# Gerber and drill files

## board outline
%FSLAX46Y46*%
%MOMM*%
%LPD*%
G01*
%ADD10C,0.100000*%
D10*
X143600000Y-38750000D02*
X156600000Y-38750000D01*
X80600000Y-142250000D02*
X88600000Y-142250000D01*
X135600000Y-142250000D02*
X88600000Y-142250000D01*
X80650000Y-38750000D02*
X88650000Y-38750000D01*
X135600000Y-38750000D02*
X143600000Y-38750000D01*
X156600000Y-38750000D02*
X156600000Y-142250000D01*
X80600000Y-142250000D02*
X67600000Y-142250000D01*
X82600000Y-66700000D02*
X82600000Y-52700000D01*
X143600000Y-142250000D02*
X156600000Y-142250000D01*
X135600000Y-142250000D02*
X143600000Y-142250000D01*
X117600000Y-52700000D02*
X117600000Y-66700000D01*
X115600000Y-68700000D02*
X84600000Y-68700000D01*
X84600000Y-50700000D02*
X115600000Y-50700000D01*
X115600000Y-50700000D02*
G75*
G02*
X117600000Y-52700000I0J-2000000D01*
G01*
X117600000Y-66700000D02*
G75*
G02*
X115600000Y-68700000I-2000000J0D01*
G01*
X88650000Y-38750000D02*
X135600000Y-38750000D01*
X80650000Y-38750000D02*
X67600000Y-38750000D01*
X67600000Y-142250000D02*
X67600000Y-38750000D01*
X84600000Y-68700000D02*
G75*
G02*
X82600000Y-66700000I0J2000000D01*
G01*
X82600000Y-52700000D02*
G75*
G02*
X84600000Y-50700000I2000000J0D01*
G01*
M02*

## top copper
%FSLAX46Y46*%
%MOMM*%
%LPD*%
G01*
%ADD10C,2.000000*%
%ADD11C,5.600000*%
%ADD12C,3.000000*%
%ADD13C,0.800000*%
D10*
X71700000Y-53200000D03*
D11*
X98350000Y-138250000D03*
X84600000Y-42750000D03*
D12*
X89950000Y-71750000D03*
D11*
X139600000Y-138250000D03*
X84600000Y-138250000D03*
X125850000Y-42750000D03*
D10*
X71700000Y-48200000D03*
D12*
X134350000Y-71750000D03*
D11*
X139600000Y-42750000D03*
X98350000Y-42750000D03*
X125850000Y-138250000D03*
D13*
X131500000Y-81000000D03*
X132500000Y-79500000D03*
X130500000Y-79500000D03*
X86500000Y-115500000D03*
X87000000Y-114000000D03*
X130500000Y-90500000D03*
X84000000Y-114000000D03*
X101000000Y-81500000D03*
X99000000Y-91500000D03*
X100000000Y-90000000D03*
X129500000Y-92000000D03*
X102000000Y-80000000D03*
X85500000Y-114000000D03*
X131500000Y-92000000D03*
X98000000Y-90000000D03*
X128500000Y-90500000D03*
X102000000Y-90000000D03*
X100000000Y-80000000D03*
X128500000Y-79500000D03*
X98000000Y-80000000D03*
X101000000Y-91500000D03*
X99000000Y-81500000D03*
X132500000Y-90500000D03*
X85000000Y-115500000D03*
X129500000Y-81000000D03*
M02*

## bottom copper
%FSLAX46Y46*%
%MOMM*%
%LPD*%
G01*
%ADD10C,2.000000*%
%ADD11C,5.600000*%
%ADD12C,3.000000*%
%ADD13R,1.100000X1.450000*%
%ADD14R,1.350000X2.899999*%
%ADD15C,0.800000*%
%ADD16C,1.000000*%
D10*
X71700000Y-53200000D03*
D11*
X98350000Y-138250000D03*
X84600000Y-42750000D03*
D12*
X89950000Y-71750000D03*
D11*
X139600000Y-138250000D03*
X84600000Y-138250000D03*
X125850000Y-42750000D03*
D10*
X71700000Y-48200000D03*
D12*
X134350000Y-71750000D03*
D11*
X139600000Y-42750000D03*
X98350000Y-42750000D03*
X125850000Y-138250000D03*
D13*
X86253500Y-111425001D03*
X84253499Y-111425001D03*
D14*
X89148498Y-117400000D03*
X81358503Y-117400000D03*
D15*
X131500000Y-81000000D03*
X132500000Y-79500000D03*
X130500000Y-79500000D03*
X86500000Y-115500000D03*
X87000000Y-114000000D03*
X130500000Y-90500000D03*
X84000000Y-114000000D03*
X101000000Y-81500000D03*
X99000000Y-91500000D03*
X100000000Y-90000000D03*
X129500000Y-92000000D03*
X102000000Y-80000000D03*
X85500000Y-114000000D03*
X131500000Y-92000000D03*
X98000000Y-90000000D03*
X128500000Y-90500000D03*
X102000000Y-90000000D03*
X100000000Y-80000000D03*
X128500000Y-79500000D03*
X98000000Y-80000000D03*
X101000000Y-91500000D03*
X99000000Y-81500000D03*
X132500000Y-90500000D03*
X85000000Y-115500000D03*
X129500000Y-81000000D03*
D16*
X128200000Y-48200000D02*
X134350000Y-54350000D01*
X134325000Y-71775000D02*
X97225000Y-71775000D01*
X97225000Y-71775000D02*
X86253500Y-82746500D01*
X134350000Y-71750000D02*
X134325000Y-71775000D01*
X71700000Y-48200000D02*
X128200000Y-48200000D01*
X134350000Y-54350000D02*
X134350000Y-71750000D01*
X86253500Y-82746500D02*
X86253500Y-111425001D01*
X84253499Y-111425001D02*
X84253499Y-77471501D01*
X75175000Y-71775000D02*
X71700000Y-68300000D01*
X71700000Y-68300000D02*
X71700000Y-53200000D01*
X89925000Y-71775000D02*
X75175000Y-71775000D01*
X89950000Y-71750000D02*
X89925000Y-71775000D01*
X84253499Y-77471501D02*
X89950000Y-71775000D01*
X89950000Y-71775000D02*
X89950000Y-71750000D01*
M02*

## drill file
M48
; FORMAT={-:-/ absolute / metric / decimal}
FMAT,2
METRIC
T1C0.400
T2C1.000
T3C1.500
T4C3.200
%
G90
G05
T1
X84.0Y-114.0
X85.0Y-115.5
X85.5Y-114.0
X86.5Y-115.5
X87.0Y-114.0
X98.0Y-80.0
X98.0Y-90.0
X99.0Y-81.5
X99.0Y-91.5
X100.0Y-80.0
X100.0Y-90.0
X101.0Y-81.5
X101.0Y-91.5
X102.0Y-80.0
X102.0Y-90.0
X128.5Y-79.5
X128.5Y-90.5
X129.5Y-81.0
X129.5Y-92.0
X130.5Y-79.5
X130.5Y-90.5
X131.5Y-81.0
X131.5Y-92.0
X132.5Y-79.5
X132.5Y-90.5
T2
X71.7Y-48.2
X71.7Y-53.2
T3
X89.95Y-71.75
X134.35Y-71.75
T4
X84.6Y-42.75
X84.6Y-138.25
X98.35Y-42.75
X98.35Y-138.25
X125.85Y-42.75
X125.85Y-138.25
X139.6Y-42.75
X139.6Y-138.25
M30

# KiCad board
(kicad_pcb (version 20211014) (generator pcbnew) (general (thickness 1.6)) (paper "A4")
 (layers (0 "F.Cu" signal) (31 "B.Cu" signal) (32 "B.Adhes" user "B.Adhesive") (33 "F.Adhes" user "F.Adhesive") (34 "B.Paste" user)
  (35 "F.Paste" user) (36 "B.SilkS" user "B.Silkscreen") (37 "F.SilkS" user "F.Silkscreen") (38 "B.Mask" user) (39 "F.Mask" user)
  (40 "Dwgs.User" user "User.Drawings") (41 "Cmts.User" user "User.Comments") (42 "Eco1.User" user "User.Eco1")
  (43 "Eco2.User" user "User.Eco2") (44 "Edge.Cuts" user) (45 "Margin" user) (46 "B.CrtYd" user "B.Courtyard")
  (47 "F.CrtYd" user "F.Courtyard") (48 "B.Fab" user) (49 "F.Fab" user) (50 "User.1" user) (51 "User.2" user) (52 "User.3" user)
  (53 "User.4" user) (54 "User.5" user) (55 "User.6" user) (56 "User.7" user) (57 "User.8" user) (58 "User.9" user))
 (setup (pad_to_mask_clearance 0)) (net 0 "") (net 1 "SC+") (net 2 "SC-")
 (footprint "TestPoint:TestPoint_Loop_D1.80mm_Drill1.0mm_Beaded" (layer "F.Cu") (at 71.75 53.2)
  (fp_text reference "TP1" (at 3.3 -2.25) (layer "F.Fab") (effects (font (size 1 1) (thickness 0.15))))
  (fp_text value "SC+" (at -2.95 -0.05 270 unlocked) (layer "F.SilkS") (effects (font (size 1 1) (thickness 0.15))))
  (pad "1" thru_hole circle (at -0.05 0) (size 2 2) (drill 1) (layers *.Cu *.Mask) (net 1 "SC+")))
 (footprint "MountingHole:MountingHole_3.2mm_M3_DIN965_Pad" (layer "F.Cu") (at 98.35 138.25)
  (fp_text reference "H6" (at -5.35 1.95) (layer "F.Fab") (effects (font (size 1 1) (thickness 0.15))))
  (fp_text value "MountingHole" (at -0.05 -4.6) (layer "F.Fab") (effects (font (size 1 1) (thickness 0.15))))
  (pad "1" thru_hole circle (at 0 0) (size 5.6 5.6) (drill 3.2) (layers *.Cu *.Mask)))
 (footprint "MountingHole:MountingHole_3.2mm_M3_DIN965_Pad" (layer "F.Cu") (at 84.6 42.75)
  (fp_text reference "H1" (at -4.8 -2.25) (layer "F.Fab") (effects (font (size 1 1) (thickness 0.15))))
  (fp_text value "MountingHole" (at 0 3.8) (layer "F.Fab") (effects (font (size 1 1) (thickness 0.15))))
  (pad "1" thru_hole circle (at 0 0) (size 5.6 5.6) (drill 3.2) (layers *.Cu *.Mask)))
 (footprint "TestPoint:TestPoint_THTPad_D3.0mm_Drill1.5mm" (layer "F.Cu") (at 89.95 71.75)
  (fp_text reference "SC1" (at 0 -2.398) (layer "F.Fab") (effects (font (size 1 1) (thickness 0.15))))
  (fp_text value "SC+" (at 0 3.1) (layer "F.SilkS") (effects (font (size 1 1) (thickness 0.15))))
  (pad "1" thru_hole circle (at 0 0) (size 3 3) (drill 1.5) (layers *.Cu *.Mask) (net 1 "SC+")))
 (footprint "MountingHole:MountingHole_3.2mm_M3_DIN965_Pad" (layer "F.Cu") (at 139.6 138.25)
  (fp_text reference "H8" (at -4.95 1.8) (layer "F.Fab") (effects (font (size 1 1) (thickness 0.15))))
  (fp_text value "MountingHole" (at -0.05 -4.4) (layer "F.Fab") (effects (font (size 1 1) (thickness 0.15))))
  (pad "1" thru_hole circle (at 0 0) (size 5.6 5.6) (drill 3.2) (layers *.Cu *.Mask)))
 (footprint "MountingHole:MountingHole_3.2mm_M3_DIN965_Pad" (layer "F.Cu") (at 84.6 138.25)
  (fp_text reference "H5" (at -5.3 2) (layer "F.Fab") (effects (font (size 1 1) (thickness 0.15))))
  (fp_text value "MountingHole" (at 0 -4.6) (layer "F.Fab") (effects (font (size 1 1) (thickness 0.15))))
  (pad "1" thru_hole circle (at 0 0) (size 5.6 5.6) (drill 3.2) (layers *.Cu *.Mask)))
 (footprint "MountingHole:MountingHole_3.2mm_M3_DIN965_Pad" (layer "F.Cu") (at 125.85 42.75)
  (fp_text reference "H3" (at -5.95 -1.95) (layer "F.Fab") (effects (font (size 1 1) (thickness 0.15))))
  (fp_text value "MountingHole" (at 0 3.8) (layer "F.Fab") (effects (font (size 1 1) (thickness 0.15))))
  (pad "1" thru_hole circle (at 0 0) (size 5.6 5.6) (drill 3.2) (layers *.Cu *.Mask)))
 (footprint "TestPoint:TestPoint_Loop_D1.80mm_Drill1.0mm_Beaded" (layer "F.Cu") (at 71.7 48.3)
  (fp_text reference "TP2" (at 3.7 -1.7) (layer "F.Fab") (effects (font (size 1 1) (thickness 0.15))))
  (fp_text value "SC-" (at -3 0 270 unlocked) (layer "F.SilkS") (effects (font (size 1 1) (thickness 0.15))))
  (pad "1" thru_hole circle (at 0 -0.1) (size 2 2) (drill 1) (layers *.Cu *.Mask) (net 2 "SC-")))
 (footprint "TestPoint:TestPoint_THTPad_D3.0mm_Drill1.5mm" (layer "F.Cu") (at 134.35 71.75)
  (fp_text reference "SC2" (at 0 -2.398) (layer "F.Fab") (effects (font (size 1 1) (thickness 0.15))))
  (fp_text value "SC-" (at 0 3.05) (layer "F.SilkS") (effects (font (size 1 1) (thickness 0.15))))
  (pad "1" thru_hole circle (at 0 0) (size 3 3) (drill 1.5) (layers *.Cu *.Mask) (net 2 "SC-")))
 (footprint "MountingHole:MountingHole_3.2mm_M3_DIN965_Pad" (layer "F.Cu") (at 139.6 42.75)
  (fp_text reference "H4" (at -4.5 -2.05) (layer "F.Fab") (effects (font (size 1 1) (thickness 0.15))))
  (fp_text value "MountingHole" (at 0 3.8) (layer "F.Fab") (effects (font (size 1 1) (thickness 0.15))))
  (pad "1" thru_hole circle (at 0 0) (size 5.6 5.6) (drill 3.2) (layers *.Cu *.Mask)))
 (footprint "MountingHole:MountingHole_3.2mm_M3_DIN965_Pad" (layer "F.Cu") (at 98.35 42.75)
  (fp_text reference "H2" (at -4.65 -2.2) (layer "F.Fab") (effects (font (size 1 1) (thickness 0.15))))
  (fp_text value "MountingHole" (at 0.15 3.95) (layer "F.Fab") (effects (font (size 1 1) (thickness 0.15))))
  (pad "1" thru_hole circle (at 0 0) (size 5.6 5.6) (drill 3.2) (layers *.Cu *.Mask)))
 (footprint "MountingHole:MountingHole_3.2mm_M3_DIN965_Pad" (layer "F.Cu") (at 125.85 138.25)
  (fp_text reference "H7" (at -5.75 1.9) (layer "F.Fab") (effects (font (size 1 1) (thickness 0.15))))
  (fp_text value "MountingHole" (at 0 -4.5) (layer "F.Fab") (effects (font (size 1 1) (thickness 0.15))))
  (pad "1" thru_hole circle (at 0 0) (size 5.6 5.6) (drill 3.2) (layers *.Cu *.Mask)))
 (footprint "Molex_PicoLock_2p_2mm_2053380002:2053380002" (layer "B.Cu") (at 86.2535 111.425001)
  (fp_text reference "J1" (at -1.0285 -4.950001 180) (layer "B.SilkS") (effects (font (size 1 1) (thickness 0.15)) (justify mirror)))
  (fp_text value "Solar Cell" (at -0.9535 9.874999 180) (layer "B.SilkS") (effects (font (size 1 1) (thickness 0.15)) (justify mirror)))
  (pad "1" smd rect (at 0 0) (size 1.1 1.45) (layers "B.Cu" "B.Paste" "B.Mask") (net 2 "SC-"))
  (pad "2" smd rect (at -2.000001 0) (size 1.1 1.45) (layers "B.Cu" "B.Paste" "B.Mask") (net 1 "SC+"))
  (pad "3" smd rect (at 2.894998 5.974999) (size 1.35 2.899999) (layers "B.Cu" "B.Paste" "B.Mask"))
  (pad "4" smd rect (at -4.894997 5.974999) (size 1.35 2.899999) (layers "B.Cu" "B.Paste" "B.Mask")))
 (gr_line (start 143.6 38.75) (end 156.6 38.75) (layer "Edge.Cuts") (width 0.1))
 (gr_line (start 80.6 142.25) (end 88.6 142.25) (layer "Edge.Cuts") (width 0.1))
 (gr_line (start 135.6 142.25) (end 88.6 142.25) (layer "Edge.Cuts") (width 0.1))
 (gr_line (start 80.65 38.75) (end 88.65 38.75) (layer "Edge.Cuts") (width 0.1))
 (gr_line (start 135.6 38.75) (end 143.6 38.75) (layer "Edge.Cuts") (width 0.1))
 (gr_line (start 156.6 38.75) (end 156.6 142.25) (layer "Edge.Cuts") (width 0.1))
 (gr_line (start 80.6 142.25) (end 67.6 142.25) (layer "Edge.Cuts") (width 0.1))
 (gr_line (start 82.6 66.7) (end 82.6 52.7) (layer "Edge.Cuts") (width 0.1))
 (gr_line (start 143.6 142.25) (end 156.6 142.25) (layer "Edge.Cuts") (width 0.1))
 (gr_line (start 135.6 142.25) (end 143.6 142.25) (layer "Edge.Cuts") (width 0.1))
 (gr_line (start 117.6 52.7) (end 117.6 66.7) (layer "Edge.Cuts") (width 0.1))
 (gr_line (start 115.6 68.7) (end 84.6 68.7) (layer "Edge.Cuts") (width 0.1))
 (gr_line (start 84.6 50.7) (end 115.6 50.7) (layer "Edge.Cuts") (width 0.1))
 (gr_arc (start 115.6 50.7) (mid 117.014214 51.285786) (end 117.6 52.7) (layer "Edge.Cuts") (width 0.1))
 (gr_arc (start 117.6 66.7) (mid 117.014214 68.114214) (end 115.6 68.7) (layer "Edge.Cuts") (width 0.1))
 (gr_line (start 88.65 38.75) (end 135.6 38.75) (layer "Edge.Cuts") (width 0.1))
 (gr_line (start 80.65 38.75) (end 67.6 38.75) (layer "Edge.Cuts") (width 0.1))
 (gr_line (start 67.6 142.25) (end 67.6 38.75) (layer "Edge.Cuts") (width 0.1))
 (gr_arc (start 84.6 68.7) (mid 83.185786 68.114214) (end 82.6 66.7) (layer "Edge.Cuts") (width 0.1))
 (gr_arc (start 82.6 52.7) (mid 83.185786 51.285786) (end 84.6 50.7) (layer "Edge.Cuts") (width 0.1))
 (via (at 131.5 81) (size 0.8) (drill 0.4) (layers "F.Cu" "B.Cu") (free) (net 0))
 (via (at 132.5 79.5) (size 0.8) (drill 0.4) (layers "F.Cu" "B.Cu") (free) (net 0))
 (via (at 130.5 79.5) (size 0.8) (drill 0.4) (layers "F.Cu" "B.Cu") (free) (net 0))
 (via (at 86.5 115.5) (size 0.8) (drill 0.4) (layers "F.Cu" "B.Cu") (free) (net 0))
 (via (at 87 114) (size 0.8) (drill 0.4) (layers "F.Cu" "B.Cu") (free) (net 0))
 (via (at 130.5 90.5) (size 0.8) (drill 0.4) (layers "F.Cu" "B.Cu") (free) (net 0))
 (via (at 84 114) (size 0.8) (drill 0.4) (layers "F.Cu" "B.Cu") (free) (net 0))
 (via (at 101 81.5) (size 0.8) (drill 0.4) (layers "F.Cu" "B.Cu") (free) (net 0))
 (via (at 99 91.5) (size 0.8) (drill 0.4) (layers "F.Cu" "B.Cu") (free) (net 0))
 (via (at 100 90) (size 0.8) (drill 0.4) (layers "F.Cu" "B.Cu") (free) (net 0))
 (via (at 129.5 92) (size 0.8) (drill 0.4) (layers "F.Cu" "B.Cu") (free) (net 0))
 (via (at 102 80) (size 0.8) (drill 0.4) (layers "F.Cu" "B.Cu") (free) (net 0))
 (via (at 85.5 114) (size 0.8) (drill 0.4) (layers "F.Cu" "B.Cu") (free) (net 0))
 (via (at 131.5 92) (size 0.8) (drill 0.4) (layers "F.Cu" "B.Cu") (free) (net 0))
 (via (at 98 90) (size 0.8) (drill 0.4) (layers "F.Cu" "B.Cu") (free) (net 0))
 (via (at 128.5 90.5) (size 0.8) (drill 0.4) (layers "F.Cu" "B.Cu") (free) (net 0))
 (via (at 102 90) (size 0.8) (drill 0.4) (layers "F.Cu" "B.Cu") (free) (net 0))
 (via (at 100 80) (size 0.8) (drill 0.4) (layers "F.Cu" "B.Cu") (free) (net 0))
 (via (at 128.5 79.5) (size 0.8) (drill 0.4) (layers "F.Cu" "B.Cu") (free) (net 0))
 (via (at 98 80) (size 0.8) (drill 0.4) (layers "F.Cu" "B.Cu") (free) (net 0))
 (via (at 101 91.5) (size 0.8) (drill 0.4) (layers "F.Cu" "B.Cu") (free) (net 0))
 (via (at 99 81.5) (size 0.8) (drill 0.4) (layers "F.Cu" "B.Cu") (free) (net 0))
 (via (at 132.5 90.5) (size 0.8) (drill 0.4) (layers "F.Cu" "B.Cu") (free) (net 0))
 (via (at 85 115.5) (size 0.8) (drill 0.4) (layers "F.Cu" "B.Cu") (free) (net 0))
 (via (at 129.5 81) (size 0.8) (drill 0.4) (layers "F.Cu" "B.Cu") (free) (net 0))
 (segment (start 128.2 48.2) (end 134.35 54.35) (width 1) (layer "B.Cu") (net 2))
 (segment (start 134.325 71.775) (end 97.225 71.775) (width 1) (layer "B.Cu") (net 2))
 (segment (start 97.225 71.775) (end 86.2535 82.7465) (width 1) (layer "B.Cu") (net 2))
 (segment (start 134.35 71.75) (end 134.325 71.775) (width 1) (layer "B.Cu") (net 2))
 (segment (start 71.7 48.2) (end 128.2 48.2) (width 1) (layer "B.Cu") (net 2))
 (segment (start 134.35 54.35) (end 134.35 71.75) (width 1) (layer "B.Cu") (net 2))
 (segment (start 86.2535 82.7465) (end 86.2535 111.425001) (width 1) (layer "B.Cu") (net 2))
 (segment (start 84.253499 111.425001) (end 84.253499 77.471501) (width 1) (layer "B.Cu") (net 1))
 (segment (start 75.175 71.775) (end 71.7 68.3) (width 1) (layer "B.Cu") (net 1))
 (segment (start 71.7 68.3) (end 71.7 53.2) (width 1) (layer "B.Cu") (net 1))
 (segment (start 89.925 71.775) (end 75.175 71.775) (width 1) (layer "B.Cu") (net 1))
 (segment (start 89.95 71.75) (end 89.925 71.775) (width 1) (layer "B.Cu") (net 1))
 (segment (start 84.253499 77.471501) (end 89.95 71.775) (width 1) (layer "B.Cu") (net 1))
 (segment (start 89.95 71.775) (end 89.95 71.75) (width 1) (layer "B.Cu") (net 1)))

